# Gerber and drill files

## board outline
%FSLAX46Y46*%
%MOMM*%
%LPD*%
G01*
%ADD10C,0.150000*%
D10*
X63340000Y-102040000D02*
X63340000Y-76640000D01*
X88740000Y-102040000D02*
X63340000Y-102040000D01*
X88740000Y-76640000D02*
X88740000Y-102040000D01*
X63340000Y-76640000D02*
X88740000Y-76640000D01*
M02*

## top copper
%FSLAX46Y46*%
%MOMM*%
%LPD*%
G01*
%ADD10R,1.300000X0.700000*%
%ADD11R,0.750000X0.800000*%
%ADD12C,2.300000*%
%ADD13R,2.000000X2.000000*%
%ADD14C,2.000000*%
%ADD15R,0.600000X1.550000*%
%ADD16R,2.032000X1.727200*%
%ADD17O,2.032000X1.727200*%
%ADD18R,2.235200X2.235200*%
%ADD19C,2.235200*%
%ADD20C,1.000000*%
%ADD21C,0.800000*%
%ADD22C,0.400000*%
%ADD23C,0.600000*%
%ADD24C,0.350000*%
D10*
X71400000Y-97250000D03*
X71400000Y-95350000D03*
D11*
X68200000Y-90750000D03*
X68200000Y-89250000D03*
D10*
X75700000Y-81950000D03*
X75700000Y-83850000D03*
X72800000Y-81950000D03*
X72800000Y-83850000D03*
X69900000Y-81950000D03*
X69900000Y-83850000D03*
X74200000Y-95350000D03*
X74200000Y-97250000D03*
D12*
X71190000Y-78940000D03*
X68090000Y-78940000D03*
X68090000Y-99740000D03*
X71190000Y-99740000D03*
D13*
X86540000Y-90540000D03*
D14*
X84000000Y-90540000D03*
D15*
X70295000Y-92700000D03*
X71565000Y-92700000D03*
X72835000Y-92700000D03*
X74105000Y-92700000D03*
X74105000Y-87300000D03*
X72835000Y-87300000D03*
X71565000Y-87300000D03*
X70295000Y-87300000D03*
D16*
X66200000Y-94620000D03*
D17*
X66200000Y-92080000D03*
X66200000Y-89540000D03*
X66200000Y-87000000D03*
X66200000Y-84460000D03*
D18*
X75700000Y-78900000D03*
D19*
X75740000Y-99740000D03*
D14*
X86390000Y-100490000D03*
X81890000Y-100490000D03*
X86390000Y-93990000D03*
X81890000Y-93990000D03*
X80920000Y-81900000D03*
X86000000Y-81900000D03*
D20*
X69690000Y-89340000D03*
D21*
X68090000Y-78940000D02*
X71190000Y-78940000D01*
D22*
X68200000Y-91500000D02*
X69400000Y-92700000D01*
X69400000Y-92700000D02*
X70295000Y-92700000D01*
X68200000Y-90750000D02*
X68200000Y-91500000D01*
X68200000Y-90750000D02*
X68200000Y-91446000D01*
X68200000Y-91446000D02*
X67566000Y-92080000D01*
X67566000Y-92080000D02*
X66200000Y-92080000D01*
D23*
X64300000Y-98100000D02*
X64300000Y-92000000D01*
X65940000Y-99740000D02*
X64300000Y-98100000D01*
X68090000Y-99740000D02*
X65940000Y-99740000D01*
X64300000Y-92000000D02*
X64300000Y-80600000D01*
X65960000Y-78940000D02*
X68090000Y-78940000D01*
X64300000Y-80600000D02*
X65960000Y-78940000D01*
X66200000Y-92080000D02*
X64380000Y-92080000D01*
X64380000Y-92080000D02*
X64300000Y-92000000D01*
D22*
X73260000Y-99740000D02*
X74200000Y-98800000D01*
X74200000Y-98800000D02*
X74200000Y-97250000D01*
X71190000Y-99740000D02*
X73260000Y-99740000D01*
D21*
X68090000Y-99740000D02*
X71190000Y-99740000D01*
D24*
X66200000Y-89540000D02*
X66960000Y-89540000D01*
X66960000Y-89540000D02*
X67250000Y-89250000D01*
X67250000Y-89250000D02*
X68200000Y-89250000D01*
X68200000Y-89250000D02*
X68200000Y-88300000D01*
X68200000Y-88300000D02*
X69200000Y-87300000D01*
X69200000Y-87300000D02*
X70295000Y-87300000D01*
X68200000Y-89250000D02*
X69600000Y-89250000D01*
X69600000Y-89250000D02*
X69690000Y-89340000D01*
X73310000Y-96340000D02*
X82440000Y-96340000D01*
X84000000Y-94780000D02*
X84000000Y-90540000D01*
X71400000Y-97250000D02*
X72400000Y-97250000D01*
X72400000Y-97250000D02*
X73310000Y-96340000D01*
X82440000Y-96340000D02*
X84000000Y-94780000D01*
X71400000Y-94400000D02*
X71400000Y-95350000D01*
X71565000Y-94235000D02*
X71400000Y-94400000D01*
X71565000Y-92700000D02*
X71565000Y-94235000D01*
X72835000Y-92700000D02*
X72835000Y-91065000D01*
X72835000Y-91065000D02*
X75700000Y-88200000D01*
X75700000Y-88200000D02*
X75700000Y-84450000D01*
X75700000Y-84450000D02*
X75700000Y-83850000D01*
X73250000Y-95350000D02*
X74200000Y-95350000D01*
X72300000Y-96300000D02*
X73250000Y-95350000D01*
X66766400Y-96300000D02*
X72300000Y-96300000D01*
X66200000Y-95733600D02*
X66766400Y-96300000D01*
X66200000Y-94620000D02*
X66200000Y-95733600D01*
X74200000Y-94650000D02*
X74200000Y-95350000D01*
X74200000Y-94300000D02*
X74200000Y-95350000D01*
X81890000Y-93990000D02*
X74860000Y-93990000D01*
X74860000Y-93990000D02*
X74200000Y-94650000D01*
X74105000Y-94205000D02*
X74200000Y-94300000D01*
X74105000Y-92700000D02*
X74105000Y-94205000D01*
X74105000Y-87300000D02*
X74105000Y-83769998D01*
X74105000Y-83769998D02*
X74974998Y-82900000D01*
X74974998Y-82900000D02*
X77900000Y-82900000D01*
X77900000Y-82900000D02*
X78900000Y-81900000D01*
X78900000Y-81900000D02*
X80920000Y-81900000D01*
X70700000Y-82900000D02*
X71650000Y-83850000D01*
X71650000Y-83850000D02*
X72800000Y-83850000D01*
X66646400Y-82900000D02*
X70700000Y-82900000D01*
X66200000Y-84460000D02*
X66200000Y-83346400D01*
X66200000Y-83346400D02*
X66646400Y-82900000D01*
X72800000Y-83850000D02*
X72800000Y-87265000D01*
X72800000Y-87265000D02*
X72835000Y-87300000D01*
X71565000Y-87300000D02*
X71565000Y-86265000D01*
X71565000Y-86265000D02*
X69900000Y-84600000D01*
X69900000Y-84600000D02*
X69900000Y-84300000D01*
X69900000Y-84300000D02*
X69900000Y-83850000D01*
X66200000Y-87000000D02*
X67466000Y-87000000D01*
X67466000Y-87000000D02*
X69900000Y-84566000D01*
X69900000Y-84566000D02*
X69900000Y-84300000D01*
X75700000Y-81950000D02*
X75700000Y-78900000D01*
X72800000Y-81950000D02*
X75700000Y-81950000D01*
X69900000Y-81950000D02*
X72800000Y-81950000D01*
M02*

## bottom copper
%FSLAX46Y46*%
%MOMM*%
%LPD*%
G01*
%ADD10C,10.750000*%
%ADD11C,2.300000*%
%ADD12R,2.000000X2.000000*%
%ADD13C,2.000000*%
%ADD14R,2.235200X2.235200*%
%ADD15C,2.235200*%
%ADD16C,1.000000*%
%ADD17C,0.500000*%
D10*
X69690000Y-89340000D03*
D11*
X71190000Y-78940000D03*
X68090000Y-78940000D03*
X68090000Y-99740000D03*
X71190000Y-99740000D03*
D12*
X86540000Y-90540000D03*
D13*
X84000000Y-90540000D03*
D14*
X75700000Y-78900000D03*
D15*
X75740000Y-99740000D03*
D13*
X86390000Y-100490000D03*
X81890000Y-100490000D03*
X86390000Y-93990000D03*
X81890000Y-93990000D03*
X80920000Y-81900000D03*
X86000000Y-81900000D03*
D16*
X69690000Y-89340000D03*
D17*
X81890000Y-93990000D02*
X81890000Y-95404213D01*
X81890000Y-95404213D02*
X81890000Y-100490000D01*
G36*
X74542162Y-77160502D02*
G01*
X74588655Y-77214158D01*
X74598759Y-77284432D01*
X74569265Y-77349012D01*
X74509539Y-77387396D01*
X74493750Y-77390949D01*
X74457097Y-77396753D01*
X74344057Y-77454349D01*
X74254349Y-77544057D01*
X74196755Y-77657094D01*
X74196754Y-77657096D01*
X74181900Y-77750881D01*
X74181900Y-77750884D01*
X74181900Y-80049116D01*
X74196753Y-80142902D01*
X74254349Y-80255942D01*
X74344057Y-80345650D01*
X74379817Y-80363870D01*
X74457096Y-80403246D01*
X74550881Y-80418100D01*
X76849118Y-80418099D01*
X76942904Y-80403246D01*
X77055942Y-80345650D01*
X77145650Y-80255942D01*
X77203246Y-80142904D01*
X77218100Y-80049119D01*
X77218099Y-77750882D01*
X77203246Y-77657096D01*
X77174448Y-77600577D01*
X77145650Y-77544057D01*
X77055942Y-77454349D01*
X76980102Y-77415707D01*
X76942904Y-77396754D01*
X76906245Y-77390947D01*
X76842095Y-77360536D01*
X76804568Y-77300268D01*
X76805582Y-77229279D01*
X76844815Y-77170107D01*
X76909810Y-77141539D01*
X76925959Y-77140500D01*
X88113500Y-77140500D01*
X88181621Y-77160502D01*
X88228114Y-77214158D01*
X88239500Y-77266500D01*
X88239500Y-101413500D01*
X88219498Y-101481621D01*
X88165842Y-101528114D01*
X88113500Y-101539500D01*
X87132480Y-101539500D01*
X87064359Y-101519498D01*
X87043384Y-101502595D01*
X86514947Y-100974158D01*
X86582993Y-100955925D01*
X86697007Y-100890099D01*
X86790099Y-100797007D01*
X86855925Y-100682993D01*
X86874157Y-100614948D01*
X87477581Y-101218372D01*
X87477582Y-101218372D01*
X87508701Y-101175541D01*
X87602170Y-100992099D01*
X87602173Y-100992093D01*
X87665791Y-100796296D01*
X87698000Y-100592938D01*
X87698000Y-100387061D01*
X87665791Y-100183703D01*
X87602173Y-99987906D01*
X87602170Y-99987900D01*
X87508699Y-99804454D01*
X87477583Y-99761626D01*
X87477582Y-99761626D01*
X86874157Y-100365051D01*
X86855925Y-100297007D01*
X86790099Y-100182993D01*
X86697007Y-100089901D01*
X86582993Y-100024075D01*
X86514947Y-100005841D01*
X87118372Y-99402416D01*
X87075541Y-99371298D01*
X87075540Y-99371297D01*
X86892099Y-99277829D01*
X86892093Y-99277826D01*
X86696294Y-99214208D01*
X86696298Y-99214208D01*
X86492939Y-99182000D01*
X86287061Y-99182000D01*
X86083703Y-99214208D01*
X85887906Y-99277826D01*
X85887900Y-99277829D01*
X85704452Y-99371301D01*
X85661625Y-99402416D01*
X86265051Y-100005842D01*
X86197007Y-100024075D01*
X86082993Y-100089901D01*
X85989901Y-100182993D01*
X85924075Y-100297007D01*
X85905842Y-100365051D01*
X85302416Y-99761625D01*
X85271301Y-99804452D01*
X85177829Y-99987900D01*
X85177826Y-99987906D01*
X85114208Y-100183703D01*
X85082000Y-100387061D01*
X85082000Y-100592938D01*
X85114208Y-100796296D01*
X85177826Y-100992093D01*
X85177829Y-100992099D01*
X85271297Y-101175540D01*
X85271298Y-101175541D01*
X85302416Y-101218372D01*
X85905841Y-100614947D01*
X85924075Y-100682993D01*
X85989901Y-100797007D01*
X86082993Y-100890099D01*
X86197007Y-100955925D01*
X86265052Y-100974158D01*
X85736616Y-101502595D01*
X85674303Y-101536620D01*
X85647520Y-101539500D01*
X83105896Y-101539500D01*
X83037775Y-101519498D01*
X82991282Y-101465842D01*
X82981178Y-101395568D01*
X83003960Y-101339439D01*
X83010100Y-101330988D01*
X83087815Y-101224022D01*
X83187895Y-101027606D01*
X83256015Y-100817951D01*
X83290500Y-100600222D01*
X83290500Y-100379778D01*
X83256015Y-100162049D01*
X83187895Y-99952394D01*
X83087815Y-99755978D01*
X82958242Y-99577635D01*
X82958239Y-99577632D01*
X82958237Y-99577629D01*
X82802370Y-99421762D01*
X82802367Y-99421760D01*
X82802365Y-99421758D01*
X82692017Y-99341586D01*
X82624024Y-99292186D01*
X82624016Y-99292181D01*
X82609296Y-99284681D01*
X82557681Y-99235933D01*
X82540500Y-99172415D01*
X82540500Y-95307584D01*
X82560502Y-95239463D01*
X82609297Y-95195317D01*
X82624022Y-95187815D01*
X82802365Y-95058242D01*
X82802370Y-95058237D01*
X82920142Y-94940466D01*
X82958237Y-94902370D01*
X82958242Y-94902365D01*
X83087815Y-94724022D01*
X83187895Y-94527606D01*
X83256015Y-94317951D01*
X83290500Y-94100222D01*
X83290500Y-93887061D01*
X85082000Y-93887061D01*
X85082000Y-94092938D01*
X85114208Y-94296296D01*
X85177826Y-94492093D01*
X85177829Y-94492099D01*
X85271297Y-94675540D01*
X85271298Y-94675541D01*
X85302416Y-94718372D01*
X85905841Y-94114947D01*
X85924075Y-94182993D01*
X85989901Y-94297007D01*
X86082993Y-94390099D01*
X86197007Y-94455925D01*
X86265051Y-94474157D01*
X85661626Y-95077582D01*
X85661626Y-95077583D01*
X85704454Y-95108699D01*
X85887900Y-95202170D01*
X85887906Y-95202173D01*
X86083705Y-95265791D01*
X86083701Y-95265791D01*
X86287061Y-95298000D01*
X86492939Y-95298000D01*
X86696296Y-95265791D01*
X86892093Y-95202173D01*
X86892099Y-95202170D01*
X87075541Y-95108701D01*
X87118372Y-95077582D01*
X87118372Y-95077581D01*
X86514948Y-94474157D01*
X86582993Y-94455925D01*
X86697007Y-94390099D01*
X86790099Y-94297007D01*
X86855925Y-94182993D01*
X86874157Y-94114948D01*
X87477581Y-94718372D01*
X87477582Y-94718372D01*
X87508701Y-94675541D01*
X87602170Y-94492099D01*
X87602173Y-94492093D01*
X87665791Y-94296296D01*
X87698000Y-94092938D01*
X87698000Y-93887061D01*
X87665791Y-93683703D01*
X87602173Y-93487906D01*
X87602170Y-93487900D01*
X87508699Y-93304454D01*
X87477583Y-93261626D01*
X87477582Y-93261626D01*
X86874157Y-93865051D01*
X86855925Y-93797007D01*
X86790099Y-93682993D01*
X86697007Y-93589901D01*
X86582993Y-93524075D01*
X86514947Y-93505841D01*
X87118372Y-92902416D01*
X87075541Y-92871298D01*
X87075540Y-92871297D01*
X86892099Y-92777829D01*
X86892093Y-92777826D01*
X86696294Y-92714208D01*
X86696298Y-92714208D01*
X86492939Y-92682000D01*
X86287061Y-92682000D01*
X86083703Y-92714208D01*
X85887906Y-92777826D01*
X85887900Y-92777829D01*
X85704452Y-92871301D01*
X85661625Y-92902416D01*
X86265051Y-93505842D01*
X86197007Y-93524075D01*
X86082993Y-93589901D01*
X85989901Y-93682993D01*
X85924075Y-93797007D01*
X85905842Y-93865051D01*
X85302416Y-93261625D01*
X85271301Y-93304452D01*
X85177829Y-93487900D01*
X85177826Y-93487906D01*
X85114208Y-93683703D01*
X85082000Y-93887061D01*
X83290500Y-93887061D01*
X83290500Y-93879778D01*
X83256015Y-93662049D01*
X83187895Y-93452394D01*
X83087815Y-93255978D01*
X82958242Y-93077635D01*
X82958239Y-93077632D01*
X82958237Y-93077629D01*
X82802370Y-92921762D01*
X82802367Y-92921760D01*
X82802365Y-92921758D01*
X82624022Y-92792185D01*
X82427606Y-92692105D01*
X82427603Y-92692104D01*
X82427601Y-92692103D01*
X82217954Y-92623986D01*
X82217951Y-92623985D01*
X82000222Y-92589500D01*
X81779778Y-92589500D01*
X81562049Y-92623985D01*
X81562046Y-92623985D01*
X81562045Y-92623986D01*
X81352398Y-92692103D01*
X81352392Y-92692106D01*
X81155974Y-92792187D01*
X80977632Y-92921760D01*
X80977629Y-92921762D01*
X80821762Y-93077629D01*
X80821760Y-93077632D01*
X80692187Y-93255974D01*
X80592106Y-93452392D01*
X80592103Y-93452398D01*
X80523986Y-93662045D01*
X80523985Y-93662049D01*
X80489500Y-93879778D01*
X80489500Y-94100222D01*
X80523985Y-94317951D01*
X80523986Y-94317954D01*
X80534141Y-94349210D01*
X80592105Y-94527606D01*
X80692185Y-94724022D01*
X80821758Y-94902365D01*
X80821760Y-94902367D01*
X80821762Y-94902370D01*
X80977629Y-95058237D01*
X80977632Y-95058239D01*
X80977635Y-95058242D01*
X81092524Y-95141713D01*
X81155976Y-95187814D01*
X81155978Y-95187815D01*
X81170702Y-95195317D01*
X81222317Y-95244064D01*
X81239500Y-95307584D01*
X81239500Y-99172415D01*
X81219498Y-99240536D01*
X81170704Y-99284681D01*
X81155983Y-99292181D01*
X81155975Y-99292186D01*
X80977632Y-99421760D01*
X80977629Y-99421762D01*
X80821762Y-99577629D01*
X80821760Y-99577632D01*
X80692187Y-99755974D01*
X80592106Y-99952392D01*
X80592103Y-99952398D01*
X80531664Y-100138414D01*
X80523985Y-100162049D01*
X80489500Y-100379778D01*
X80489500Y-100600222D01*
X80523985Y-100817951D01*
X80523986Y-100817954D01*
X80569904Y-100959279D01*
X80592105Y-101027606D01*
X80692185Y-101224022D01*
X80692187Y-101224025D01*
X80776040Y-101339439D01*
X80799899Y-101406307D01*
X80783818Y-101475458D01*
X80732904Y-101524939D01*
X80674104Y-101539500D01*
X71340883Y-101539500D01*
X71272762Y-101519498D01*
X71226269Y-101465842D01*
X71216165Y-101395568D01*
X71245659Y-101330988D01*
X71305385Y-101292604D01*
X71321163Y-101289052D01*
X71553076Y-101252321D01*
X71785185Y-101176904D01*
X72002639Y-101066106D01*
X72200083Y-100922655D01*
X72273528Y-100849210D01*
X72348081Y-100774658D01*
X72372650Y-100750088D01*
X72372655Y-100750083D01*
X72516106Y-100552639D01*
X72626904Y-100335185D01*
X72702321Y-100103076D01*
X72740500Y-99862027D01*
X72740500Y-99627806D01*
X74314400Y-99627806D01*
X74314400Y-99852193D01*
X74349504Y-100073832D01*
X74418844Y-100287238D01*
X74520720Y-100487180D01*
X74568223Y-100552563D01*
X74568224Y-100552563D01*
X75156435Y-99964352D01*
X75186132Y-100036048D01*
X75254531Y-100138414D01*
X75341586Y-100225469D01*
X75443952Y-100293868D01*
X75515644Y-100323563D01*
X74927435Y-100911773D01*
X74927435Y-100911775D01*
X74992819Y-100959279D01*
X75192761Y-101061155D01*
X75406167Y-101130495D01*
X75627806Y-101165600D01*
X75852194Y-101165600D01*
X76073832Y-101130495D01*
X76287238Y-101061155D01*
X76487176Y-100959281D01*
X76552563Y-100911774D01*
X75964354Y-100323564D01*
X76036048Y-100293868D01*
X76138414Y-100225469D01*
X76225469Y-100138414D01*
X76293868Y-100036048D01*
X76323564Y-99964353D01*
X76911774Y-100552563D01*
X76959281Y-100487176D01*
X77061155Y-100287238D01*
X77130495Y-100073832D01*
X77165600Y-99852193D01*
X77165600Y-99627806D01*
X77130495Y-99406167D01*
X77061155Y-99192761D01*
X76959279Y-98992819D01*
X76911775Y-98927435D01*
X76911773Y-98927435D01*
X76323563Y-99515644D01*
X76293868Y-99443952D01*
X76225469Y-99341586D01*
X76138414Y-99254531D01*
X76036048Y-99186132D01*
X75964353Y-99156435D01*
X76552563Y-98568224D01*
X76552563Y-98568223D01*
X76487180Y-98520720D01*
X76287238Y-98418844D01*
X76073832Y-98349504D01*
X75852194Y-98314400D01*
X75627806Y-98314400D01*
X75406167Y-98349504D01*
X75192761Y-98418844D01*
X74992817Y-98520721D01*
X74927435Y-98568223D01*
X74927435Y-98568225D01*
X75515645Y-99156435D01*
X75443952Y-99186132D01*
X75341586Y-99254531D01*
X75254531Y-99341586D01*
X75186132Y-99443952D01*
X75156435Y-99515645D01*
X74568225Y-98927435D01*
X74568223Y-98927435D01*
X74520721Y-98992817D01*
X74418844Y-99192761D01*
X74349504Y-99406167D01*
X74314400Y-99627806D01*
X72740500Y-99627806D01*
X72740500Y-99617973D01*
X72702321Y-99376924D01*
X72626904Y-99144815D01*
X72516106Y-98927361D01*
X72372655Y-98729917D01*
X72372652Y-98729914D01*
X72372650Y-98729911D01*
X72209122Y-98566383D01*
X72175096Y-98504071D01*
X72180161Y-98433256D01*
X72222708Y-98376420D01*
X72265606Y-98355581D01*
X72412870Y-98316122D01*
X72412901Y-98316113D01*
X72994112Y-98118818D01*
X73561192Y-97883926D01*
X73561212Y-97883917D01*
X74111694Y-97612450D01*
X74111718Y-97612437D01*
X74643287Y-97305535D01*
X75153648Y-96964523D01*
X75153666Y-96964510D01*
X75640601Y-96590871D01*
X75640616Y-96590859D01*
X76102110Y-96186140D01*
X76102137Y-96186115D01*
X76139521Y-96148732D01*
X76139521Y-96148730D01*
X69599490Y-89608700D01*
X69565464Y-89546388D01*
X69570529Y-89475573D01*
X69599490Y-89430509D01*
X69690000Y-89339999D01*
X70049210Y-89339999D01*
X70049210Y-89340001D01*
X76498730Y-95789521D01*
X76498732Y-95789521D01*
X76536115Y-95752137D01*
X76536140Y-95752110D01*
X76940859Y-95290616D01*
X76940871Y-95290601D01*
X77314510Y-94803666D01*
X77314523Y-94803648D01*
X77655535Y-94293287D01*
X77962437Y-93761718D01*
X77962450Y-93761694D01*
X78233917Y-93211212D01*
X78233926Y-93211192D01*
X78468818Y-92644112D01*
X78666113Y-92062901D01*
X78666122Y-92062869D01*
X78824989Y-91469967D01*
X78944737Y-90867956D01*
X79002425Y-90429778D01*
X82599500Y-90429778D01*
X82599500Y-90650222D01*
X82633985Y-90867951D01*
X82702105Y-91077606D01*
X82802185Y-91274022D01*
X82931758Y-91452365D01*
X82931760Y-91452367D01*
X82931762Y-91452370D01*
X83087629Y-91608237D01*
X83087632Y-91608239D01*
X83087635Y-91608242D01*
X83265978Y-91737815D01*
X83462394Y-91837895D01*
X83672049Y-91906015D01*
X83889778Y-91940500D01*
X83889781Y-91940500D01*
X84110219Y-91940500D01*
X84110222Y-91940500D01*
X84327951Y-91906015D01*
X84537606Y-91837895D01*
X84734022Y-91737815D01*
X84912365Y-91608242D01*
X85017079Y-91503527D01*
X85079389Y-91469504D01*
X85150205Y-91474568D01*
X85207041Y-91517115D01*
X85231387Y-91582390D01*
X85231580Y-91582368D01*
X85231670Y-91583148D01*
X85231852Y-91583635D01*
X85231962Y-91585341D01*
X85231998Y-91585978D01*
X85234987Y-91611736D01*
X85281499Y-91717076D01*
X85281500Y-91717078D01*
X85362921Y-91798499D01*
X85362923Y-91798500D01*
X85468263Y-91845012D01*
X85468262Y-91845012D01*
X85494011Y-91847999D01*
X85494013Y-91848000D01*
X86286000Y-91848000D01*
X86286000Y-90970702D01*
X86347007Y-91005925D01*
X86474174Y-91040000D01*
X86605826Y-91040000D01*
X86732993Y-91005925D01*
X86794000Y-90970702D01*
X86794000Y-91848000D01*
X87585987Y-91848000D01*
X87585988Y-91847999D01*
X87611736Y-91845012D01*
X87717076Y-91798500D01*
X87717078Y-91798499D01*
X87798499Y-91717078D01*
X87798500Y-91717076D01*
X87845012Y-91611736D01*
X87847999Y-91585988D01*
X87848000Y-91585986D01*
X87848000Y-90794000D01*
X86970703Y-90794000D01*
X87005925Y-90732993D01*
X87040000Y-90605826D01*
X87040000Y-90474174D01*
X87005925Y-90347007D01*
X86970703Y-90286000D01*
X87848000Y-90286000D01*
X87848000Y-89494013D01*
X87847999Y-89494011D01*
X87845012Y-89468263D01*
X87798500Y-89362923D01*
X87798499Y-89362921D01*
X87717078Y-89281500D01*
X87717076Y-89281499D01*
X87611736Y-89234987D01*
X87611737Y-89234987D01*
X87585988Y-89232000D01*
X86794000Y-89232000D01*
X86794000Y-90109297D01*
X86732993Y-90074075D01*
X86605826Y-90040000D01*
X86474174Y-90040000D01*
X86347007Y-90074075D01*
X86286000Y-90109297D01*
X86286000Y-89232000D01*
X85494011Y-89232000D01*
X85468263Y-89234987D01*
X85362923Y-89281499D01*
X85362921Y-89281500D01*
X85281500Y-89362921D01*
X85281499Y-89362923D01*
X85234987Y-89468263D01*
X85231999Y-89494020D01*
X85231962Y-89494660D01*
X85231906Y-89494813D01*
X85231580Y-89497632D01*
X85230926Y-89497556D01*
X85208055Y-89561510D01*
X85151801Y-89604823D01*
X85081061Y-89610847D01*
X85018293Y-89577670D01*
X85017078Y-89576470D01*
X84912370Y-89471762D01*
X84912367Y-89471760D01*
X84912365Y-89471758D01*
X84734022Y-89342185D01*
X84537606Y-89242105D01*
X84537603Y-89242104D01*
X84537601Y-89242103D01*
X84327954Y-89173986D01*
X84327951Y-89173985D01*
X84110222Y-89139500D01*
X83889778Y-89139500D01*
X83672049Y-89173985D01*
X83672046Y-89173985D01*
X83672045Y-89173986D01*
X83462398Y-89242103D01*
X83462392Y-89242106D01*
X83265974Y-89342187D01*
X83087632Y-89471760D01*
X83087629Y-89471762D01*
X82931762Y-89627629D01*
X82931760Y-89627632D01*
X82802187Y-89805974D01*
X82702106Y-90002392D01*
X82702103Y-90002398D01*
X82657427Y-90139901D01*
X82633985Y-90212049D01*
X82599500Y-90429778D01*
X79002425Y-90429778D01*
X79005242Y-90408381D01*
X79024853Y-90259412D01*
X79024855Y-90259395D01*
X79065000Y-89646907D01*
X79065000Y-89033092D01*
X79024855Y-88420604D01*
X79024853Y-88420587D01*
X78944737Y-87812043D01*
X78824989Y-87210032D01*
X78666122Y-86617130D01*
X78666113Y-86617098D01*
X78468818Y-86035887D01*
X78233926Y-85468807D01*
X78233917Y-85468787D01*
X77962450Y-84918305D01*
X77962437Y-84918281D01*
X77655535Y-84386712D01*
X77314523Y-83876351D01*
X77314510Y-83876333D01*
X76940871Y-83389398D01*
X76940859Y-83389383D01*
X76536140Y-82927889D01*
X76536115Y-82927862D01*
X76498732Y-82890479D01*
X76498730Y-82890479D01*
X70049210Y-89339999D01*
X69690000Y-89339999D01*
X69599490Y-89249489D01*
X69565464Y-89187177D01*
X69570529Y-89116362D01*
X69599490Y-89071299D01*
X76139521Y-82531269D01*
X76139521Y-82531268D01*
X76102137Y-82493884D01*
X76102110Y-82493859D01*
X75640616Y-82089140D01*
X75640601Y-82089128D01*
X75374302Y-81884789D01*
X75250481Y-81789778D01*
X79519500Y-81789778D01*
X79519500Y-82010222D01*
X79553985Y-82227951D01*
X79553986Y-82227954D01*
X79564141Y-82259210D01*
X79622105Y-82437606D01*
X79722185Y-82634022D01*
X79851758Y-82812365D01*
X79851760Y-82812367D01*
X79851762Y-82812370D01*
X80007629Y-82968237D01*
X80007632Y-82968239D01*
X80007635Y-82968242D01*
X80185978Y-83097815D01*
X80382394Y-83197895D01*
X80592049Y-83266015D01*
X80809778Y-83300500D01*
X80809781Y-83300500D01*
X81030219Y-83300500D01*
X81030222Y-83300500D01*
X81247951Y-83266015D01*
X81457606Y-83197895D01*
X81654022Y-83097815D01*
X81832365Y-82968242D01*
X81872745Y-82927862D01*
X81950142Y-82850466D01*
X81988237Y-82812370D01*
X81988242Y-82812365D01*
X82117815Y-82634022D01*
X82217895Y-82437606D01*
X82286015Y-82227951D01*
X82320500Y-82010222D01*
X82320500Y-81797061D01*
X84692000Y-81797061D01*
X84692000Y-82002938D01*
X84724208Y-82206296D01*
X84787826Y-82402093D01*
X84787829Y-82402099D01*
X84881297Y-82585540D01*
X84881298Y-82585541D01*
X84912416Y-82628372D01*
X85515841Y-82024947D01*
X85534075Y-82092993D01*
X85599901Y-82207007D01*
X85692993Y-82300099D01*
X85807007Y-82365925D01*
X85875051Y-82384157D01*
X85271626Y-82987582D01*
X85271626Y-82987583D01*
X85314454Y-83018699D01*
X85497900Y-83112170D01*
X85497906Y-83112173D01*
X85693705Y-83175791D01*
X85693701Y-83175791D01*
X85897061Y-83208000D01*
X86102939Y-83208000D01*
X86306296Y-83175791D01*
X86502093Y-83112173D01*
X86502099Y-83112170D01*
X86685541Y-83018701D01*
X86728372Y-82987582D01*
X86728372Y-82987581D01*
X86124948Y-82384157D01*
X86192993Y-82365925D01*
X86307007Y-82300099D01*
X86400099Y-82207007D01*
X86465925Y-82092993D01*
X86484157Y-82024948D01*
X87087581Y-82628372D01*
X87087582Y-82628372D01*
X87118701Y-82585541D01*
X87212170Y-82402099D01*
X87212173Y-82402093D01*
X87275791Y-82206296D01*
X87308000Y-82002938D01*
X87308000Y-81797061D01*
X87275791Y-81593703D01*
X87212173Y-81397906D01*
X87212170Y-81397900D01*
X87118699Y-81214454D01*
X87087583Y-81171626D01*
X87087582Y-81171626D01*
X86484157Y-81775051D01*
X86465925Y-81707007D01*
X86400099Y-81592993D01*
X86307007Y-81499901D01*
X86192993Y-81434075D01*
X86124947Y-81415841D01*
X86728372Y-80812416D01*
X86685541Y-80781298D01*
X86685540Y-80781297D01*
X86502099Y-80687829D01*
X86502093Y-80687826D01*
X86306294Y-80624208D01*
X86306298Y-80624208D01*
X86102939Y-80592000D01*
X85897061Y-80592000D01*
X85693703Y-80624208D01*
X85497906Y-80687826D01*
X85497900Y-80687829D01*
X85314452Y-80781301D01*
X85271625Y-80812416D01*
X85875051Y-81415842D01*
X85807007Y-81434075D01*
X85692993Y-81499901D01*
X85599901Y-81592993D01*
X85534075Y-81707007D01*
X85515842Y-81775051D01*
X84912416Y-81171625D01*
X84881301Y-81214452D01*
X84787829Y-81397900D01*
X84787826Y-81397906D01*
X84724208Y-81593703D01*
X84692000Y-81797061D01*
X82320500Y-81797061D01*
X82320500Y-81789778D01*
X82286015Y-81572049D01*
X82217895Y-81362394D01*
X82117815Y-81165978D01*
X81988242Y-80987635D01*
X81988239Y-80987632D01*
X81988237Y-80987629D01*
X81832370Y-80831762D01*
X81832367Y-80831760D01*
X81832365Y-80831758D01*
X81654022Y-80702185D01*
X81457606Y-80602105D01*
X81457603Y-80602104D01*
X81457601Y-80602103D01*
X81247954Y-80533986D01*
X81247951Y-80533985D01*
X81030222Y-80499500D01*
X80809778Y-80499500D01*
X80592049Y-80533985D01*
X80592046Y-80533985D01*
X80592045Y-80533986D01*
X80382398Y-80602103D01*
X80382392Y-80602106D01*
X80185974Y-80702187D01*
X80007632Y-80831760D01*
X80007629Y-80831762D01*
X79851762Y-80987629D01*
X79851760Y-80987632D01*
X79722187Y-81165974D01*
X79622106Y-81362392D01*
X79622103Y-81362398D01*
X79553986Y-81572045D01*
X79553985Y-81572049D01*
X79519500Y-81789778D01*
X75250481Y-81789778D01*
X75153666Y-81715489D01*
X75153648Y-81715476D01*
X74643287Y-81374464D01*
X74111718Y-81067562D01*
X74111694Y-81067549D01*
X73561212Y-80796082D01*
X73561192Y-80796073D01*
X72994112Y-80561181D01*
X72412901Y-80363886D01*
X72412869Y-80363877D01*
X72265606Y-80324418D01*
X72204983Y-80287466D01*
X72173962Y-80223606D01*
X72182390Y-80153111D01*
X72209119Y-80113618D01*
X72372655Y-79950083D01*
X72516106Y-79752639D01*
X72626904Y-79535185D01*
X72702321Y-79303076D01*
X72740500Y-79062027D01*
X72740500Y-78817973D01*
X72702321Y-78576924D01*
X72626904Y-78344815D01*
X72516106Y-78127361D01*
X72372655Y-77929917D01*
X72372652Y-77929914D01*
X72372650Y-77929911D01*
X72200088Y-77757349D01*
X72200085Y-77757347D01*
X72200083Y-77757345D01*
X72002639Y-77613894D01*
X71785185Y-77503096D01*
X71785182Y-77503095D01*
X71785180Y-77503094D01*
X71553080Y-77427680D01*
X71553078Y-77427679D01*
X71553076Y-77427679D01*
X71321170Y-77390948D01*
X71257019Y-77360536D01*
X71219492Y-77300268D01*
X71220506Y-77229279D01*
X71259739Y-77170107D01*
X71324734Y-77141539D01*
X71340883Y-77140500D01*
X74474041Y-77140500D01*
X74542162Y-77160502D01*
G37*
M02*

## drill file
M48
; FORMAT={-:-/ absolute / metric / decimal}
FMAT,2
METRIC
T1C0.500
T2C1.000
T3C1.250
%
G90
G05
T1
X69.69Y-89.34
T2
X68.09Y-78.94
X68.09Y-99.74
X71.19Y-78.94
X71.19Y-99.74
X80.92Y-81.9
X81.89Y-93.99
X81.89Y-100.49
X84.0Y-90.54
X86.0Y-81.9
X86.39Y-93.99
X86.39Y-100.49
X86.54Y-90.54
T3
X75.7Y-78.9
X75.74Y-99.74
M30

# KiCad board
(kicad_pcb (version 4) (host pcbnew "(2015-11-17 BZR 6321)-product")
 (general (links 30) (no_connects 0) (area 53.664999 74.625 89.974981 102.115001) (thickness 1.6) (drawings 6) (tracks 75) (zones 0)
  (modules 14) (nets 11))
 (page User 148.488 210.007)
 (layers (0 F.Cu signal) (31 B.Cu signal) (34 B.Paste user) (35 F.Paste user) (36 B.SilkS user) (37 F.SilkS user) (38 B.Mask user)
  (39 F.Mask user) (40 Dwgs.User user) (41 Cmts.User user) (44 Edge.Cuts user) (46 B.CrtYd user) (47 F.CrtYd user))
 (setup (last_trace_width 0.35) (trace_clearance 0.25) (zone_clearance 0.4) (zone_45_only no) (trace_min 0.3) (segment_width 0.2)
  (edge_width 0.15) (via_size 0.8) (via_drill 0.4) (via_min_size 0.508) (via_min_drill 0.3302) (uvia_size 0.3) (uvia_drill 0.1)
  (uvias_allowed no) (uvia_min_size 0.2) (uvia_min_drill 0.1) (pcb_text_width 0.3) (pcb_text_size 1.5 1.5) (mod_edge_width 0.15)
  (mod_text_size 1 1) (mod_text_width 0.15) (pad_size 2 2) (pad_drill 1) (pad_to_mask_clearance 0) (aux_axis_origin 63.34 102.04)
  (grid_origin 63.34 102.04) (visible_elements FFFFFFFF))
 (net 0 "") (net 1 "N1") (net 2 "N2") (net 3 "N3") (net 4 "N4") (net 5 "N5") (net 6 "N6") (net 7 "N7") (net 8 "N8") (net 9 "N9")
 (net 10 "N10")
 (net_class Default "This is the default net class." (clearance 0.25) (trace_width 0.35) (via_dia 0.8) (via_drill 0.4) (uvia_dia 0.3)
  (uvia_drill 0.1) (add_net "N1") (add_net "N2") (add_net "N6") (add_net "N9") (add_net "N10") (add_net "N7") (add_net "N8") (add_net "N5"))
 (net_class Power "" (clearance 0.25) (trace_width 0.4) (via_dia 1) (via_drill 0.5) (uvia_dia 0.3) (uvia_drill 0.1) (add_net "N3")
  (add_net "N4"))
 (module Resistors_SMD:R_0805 (layer F.Cu) (at 71.4 96.3 90)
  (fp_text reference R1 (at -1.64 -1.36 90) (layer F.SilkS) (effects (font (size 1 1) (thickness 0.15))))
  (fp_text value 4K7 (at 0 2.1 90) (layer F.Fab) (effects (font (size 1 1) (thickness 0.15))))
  (pad 1 smd rect (at -0.95 0 90) (size 0.7 1.3) (layers F.Cu F.Paste F.Mask) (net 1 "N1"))
  (pad 2 smd rect (at 0.95 0 90) (size 0.7 1.3) (layers F.Cu F.Paste F.Mask) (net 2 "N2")))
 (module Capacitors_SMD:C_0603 (layer F.Cu) (at 68.2 90 90)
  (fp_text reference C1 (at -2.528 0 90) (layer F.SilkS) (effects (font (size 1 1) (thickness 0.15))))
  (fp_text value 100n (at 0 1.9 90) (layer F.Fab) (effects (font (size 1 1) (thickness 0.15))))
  (pad 1 smd rect (at -0.75 0 90) (size 0.8 0.75) (layers F.Cu F.Paste F.Mask) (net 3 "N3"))
  (pad 2 smd rect (at 0.75 0 90) (size 0.8 0.75) (layers F.Cu F.Paste F.Mask) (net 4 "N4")))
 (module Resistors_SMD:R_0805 (layer F.Cu) (at 75.7 82.9 270)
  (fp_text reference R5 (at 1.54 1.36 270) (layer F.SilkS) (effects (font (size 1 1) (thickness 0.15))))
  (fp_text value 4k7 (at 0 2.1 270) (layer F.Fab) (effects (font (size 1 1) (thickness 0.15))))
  (pad 1 smd rect (at -0.95 0 270) (size 0.7 1.3) (layers F.Cu F.Paste F.Mask) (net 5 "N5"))
  (pad 2 smd rect (at 0.95 0 270) (size 0.7 1.3) (layers F.Cu F.Paste F.Mask) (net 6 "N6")))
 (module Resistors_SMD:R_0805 (layer F.Cu) (at 72.8 82.9 270)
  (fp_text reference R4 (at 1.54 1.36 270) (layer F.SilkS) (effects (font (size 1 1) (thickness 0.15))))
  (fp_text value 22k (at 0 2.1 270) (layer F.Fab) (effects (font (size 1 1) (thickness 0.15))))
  (pad 1 smd rect (at -0.95 0 270) (size 0.7 1.3) (layers F.Cu F.Paste F.Mask) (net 5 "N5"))
  (pad 2 smd rect (at 0.95 0 270) (size 0.7 1.3) (layers F.Cu F.Paste F.Mask) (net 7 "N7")))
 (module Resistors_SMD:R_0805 (layer F.Cu) (at 69.9 82.9 270)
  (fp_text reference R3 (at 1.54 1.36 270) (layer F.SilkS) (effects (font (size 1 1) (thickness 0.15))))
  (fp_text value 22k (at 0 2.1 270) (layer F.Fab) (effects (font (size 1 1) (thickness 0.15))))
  (pad 1 smd rect (at -0.95 0 270) (size 0.7 1.3) (layers F.Cu F.Paste F.Mask) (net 5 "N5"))
  (pad 2 smd rect (at 0.95 0 270) (size 0.7 1.3) (layers F.Cu F.Paste F.Mask) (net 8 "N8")))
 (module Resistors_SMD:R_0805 (layer F.Cu) (at 74.2 96.3 270)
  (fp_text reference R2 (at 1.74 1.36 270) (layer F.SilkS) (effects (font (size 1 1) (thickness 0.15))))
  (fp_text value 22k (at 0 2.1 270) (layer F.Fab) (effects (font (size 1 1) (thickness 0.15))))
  (pad 1 smd rect (at -0.95 0 270) (size 0.7 1.3) (layers F.Cu F.Paste F.Mask) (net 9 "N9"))
  (pad 2 smd rect (at 0.95 0 270) (size 0.7 1.3) (layers F.Cu F.Paste F.Mask) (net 3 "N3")))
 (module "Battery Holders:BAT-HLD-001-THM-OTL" (layer B.Cu) (at 69.69 89.34 90)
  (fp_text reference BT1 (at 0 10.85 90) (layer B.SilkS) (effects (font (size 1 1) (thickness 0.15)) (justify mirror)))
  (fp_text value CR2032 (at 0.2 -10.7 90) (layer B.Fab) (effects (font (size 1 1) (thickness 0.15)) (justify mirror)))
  (pad 2 smd circle (at 0 0 90) (size 10.75 10.75) (layers B.Cu B.Mask) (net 4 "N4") (solder_mask_margin 4) (clearance 2.5) (zone_connect 1)
   (thermal_gap 4))
  (pad 1 thru_hole circle (at 10.4 1.5 90) (size 2.3 2.3) (drill 1) (layers *.Cu *.Mask B.SilkS) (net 3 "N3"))
  (pad 1 thru_hole circle (at 10.4 -1.6 90) (size 2.3 2.3) (drill 1) (layers *.Cu *.Mask B.SilkS) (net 3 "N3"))
  (pad 1 thru_hole circle (at -10.4 -1.6 90) (size 2.3 2.3) (drill 1) (layers *.Cu *.Mask B.SilkS) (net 3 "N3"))
  (pad 1 thru_hole circle (at -10.4 1.5 90) (size 2.3 2.3) (drill 1) (layers *.Cu *.Mask B.SilkS) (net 3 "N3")))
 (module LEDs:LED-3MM (layer F.Cu) (at 86.54 90.54 180)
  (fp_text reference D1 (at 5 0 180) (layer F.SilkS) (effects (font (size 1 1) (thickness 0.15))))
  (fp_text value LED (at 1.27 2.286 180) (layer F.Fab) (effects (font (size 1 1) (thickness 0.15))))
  (pad 1 thru_hole rect (at 0 0 270) (size 2 2) (drill 1) (layers *.Cu *.Mask F.SilkS) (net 4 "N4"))
  (pad 2 thru_hole circle (at 2.54 0 180) (size 2 2) (drill 1) (layers *.Cu *.Mask F.SilkS) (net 1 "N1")))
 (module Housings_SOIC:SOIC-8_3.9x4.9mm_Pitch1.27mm (layer F.Cu) (at 72.2 90 90)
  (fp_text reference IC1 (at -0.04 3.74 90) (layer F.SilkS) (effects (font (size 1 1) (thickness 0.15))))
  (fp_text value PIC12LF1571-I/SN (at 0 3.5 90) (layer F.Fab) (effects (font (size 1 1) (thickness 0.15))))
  (pad 1 smd rect (at -2.7 -1.905 90) (size 1.55 0.6) (layers F.Cu F.Paste F.Mask) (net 3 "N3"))
  (pad 2 smd rect (at -2.7 -0.635 90) (size 1.55 0.6) (layers F.Cu F.Paste F.Mask) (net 2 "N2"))
  (pad 3 smd rect (at -2.7 0.635 90) (size 1.55 0.6) (layers F.Cu F.Paste F.Mask) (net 6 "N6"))
  (pad 4 smd rect (at -2.7 1.905 90) (size 1.55 0.6) (layers F.Cu F.Paste F.Mask) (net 9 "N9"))
  (pad 5 smd rect (at 2.7 1.905 90) (size 1.55 0.6) (layers F.Cu F.Paste F.Mask) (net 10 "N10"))
  (pad 6 smd rect (at 2.7 0.635 90) (size 1.55 0.6) (layers F.Cu F.Paste F.Mask) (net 7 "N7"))
  (pad 7 smd rect (at 2.7 -0.635 90) (size 1.55 0.6) (layers F.Cu F.Paste F.Mask) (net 8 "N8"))
  (pad 8 smd rect (at 2.7 -1.905 90) (size 1.55 0.6) (layers F.Cu F.Paste F.Mask) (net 4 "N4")))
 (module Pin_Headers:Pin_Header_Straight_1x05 (layer F.Cu) (at 66.2 94.62 180)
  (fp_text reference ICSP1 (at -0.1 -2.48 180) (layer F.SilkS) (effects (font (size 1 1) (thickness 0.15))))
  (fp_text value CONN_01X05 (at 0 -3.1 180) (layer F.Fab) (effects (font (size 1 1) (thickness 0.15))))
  (pad 1 smd rect (at 0 0 180) (size 2.032 1.7272) (layers F.Cu F.Mask) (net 9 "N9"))
  (pad 2 smd oval (at 0 2.54 180) (size 2.032 1.7272) (layers F.Cu F.Mask) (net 3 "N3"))
  (pad 3 smd oval (at 0 5.08 180) (size 2.032 1.7272) (layers F.Cu F.Mask) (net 4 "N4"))
  (pad 4 smd oval (at 0 7.62 180) (size 2.032 1.7272) (layers F.Cu F.Mask) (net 8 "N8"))
  (pad 5 smd oval (at 0 10.16 180) (size 2.032 1.7272) (layers F.Cu F.Mask) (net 7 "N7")))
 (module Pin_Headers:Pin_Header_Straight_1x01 (layer F.Cu) (at 75.7 78.9)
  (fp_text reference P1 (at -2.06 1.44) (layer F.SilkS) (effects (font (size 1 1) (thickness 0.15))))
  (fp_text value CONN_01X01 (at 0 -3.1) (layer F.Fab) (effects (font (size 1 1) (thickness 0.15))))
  (pad 1 thru_hole rect (at 0 0) (size 2.2352 2.2352) (drill 1.25) (layers *.Cu *.Mask F.SilkS) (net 5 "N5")))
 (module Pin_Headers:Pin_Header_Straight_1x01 (layer F.Cu) (at 75.74 99.74)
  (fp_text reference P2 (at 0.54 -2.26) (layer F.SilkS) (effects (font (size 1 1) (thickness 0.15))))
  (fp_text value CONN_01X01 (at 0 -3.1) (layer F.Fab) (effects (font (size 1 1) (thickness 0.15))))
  (pad 1 thru_hole circle (at 0 0) (size 2.2352 2.2352) (drill 1.25) (layers *.Cu *.Mask F.SilkS) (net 4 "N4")))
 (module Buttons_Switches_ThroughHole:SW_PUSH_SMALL (layer F.Cu) (at 84.14 97.24 270)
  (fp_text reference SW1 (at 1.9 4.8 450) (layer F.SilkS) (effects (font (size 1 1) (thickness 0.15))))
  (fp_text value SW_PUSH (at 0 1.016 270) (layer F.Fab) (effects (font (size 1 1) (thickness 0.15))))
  (pad 1 thru_hole circle (at 3.25 -2.25 270) (size 2 2) (drill 1) (layers *.Cu *.Mask F.SilkS) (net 4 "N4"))
  (pad 2 thru_hole circle (at 3.25 2.25 270) (size 2 2) (drill 1) (layers *.Cu *.Mask F.SilkS) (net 9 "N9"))
  (pad 1 thru_hole circle (at -3.25 -2.25 270) (size 2 2) (drill 1) (layers *.Cu *.Mask F.SilkS) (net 4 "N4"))
  (pad 2 thru_hole circle (at -3.25 2.25 270) (size 2 2) (drill 1) (layers *.Cu *.Mask F.SilkS) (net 9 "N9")))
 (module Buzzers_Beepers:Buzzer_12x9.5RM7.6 (layer F.Cu) (at 83.44984 81.9)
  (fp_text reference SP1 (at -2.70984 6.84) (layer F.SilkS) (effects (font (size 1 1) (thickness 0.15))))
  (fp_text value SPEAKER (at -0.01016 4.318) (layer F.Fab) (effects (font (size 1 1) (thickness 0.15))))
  (pad 1 thru_hole circle (at -2.52984 0) (size 2 2) (drill 1) (layers *.Cu *.Mask F.SilkS) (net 10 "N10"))
  (pad 2 thru_hole circle (at 2.55016 0) (size 2 2) (drill 1) (layers *.Cu *.Mask F.SilkS) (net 4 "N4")))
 (gr_line (start 63.34 102.04) (end 63.34 76.64) (layer Edge.Cuts) (width 0.15))
 (gr_line (start 88.74 102.04) (end 63.34 102.04) (layer Edge.Cuts) (width 0.15))
 (gr_line (start 88.74 76.64) (end 88.74 102.04) (layer Edge.Cuts) (width 0.15))
 (gr_line (start 63.34 76.64) (end 88.74 76.64) (layer Edge.Cuts) (width 0.15))
 (segment (start 68.09 78.94) (end 71.19 78.94) (width 0.8) (layer F.Cu) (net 3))
 (segment (start 68.2 91.5) (end 69.4 92.7) (width 0.4) (layer F.Cu) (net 3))
 (segment (start 69.4 92.7) (end 70.295 92.7) (width 0.4) (layer F.Cu) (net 3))
 (segment (start 68.2 90.75) (end 68.2 91.5) (width 0.4) (layer F.Cu) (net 3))
 (segment (start 68.2 90.75) (end 68.2 91.446) (width 0.4) (layer F.Cu) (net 3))
 (segment (start 68.2 91.446) (end 67.566 92.08) (width 0.4) (layer F.Cu) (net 3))
 (segment (start 67.566 92.08) (end 66.2 92.08) (width 0.4) (layer F.Cu) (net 3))
 (segment (start 64.3 98.1) (end 64.3 92) (width 0.6) (layer F.Cu) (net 3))
 (segment (start 65.94 99.74) (end 64.3 98.1) (width 0.6) (layer F.Cu) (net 3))
 (segment (start 68.09 99.74) (end 65.94 99.74) (width 0.6) (layer F.Cu) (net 3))
 (segment (start 64.3 92) (end 64.3 80.6) (width 0.6) (layer F.Cu) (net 3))
 (segment (start 65.96 78.94) (end 68.09 78.94) (width 0.6) (layer F.Cu) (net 3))
 (segment (start 64.3 80.6) (end 65.96 78.94) (width 0.6) (layer F.Cu) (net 3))
 (segment (start 66.2 92.08) (end 64.38 92.08) (width 0.6) (layer F.Cu) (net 3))
 (segment (start 64.38 92.08) (end 64.3 92) (width 0.6) (layer F.Cu) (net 3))
 (segment (start 73.26 99.74) (end 74.2 98.8) (width 0.4) (layer F.Cu) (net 3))
 (segment (start 74.2 98.8) (end 74.2 97.25) (width 0.4) (layer F.Cu) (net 3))
 (segment (start 71.19 99.74) (end 73.26 99.74) (width 0.4) (layer F.Cu) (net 3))
 (segment (start 68.09 99.74) (end 71.19 99.74) (width 0.8) (layer F.Cu) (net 3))
 (segment (start 66.2 89.54) (end 66.96 89.54) (width 0.35) (layer F.Cu) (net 4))
 (segment (start 66.96 89.54) (end 67.25 89.25) (width 0.35) (layer F.Cu) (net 4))
 (segment (start 67.25 89.25) (end 68.2 89.25) (width 0.35) (layer F.Cu) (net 4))
 (segment (start 68.2 89.25) (end 68.2 88.3) (width 0.35) (layer F.Cu) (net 4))
 (segment (start 68.2 88.3) (end 69.2 87.3) (width 0.35) (layer F.Cu) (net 4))
 (segment (start 69.2 87.3) (end 70.295 87.3) (width 0.35) (layer F.Cu) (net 4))
 (segment (start 68.2 89.25) (end 69.6 89.25) (width 0.35) (layer F.Cu) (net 4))
 (segment (start 69.6 89.25) (end 69.69 89.34) (width 0.35) (layer F.Cu) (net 4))
 (via (at 69.69 89.34) (size 1) (drill 0.5) (layers F.Cu B.Cu) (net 4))
 (segment (start 73.31 96.34) (end 82.44 96.34) (width 0.35) (layer F.Cu) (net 1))
 (segment (start 84 94.78) (end 84 90.54) (width 0.35) (layer F.Cu) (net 1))
 (segment (start 71.4 97.25) (end 72.4 97.25) (width 0.35) (layer F.Cu) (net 1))
 (segment (start 72.4 97.25) (end 73.31 96.34) (width 0.35) (layer F.Cu) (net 1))
 (segment (start 82.44 96.34) (end 84 94.78) (width 0.35) (layer F.Cu) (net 1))
 (segment (start 71.4 94.4) (end 71.4 95.35) (width 0.35) (layer F.Cu) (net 2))
 (segment (start 71.565 94.235) (end 71.4 94.4) (width 0.35) (layer F.Cu) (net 2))
 (segment (start 71.565 92.7) (end 71.565 94.235) (width 0.35) (layer F.Cu) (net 2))
 (segment (start 72.835 92.7) (end 72.835 91.065) (width 0.35) (layer F.Cu) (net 6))
 (segment (start 72.835 91.065) (end 75.7 88.2) (width 0.35) (layer F.Cu) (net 6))
 (segment (start 75.7 88.2) (end 75.7 84.45) (width 0.35) (layer F.Cu) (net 6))
 (segment (start 75.7 84.45) (end 75.7 83.85) (width 0.35) (layer F.Cu) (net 6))
 (segment (start 73.25 95.35) (end 74.2 95.35) (width 0.35) (layer F.Cu) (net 9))
 (segment (start 72.3 96.3) (end 73.25 95.35) (width 0.35) (layer F.Cu) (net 9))
 (segment (start 66.7664 96.3) (end 72.3 96.3) (width 0.35) (layer F.Cu) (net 9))
 (segment (start 66.2 95.7336) (end 66.7664 96.3) (width 0.35) (layer F.Cu) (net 9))
 (segment (start 66.2 94.62) (end 66.2 95.7336) (width 0.35) (layer F.Cu) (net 9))
 (segment (start 74.2 94.65) (end 74.2 95.35) (width 0.35) (layer F.Cu) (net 9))
 (segment (start 74.2 94.3) (end 74.2 95.35) (width 0.35) (layer F.Cu) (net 9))
 (segment (start 81.89 93.99) (end 81.89 95.404213) (width 0.5) (layer B.Cu) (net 9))
 (segment (start 81.89 95.404213) (end 81.89 100.49) (width 0.5) (layer B.Cu) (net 9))
 (segment (start 81.89 93.99) (end 74.86 93.99) (width 0.35) (layer F.Cu) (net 9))
 (segment (start 74.86 93.99) (end 74.2 94.65) (width 0.35) (layer F.Cu) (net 9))
 (segment (start 74.105 94.205) (end 74.2 94.3) (width 0.35) (layer F.Cu) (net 9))
 (segment (start 74.105 92.7) (end 74.105 94.205) (width 0.35) (layer F.Cu) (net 9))
 (segment (start 74.105 87.3) (end 74.105 83.769998) (width 0.35) (layer F.Cu) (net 10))
 (segment (start 74.105 83.769998) (end 74.974998 82.9) (width 0.35) (layer F.Cu) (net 10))
 (segment (start 74.974998 82.9) (end 77.9 82.9) (width 0.35) (layer F.Cu) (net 10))
 (segment (start 77.9 82.9) (end 78.9 81.9) (width 0.35) (layer F.Cu) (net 10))
 (segment (start 78.9 81.9) (end 80.92 81.9) (width 0.35) (layer F.Cu) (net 10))
 (segment (start 70.7 82.9) (end 71.65 83.85) (width 0.35) (layer F.Cu) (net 7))
 (segment (start 71.65 83.85) (end 72.8 83.85) (width 0.35) (layer F.Cu) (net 7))
 (segment (start 66.6464 82.9) (end 70.7 82.9) (width 0.35) (layer F.Cu) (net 7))
 (segment (start 66.2 84.46) (end 66.2 83.3464) (width 0.35) (layer F.Cu) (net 7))
 (segment (start 66.2 83.3464) (end 66.6464 82.9) (width 0.35) (layer F.Cu) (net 7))
 (segment (start 72.8 83.85) (end 72.8 87.265) (width 0.35) (layer F.Cu) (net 7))
 (segment (start 72.8 87.265) (end 72.835 87.3) (width 0.35) (layer F.Cu) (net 7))
 (segment (start 71.565 87.3) (end 71.565 86.265) (width 0.35) (layer F.Cu) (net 8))
 (segment (start 71.565 86.265) (end 69.9 84.6) (width 0.35) (layer F.Cu) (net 8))
 (segment (start 69.9 84.6) (end 69.9 84.3) (width 0.35) (layer F.Cu) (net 8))
 (segment (start 69.9 84.3) (end 69.9 83.85) (width 0.35) (layer F.Cu) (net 8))
 (segment (start 66.2 87) (end 67.466 87) (width 0.35) (layer F.Cu) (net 8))
 (segment (start 67.466 87) (end 69.9 84.566) (width 0.35) (layer F.Cu) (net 8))
 (segment (start 69.9 84.566) (end 69.9 84.3) (width 0.35) (layer F.Cu) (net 8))
 (segment (start 75.7 81.95) (end 75.7 78.9) (width 0.35) (layer F.Cu) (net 5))
 (segment (start 72.8 81.95) (end 75.7 81.95) (width 0.35) (layer F.Cu) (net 5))
 (segment (start 69.9 81.95) (end 72.8 81.95) (width 0.35) (layer F.Cu) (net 5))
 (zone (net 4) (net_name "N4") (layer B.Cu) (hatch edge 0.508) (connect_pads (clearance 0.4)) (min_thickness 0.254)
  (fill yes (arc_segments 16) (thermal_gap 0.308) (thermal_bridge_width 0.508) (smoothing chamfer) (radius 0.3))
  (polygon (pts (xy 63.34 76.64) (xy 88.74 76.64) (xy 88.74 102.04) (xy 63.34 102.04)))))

